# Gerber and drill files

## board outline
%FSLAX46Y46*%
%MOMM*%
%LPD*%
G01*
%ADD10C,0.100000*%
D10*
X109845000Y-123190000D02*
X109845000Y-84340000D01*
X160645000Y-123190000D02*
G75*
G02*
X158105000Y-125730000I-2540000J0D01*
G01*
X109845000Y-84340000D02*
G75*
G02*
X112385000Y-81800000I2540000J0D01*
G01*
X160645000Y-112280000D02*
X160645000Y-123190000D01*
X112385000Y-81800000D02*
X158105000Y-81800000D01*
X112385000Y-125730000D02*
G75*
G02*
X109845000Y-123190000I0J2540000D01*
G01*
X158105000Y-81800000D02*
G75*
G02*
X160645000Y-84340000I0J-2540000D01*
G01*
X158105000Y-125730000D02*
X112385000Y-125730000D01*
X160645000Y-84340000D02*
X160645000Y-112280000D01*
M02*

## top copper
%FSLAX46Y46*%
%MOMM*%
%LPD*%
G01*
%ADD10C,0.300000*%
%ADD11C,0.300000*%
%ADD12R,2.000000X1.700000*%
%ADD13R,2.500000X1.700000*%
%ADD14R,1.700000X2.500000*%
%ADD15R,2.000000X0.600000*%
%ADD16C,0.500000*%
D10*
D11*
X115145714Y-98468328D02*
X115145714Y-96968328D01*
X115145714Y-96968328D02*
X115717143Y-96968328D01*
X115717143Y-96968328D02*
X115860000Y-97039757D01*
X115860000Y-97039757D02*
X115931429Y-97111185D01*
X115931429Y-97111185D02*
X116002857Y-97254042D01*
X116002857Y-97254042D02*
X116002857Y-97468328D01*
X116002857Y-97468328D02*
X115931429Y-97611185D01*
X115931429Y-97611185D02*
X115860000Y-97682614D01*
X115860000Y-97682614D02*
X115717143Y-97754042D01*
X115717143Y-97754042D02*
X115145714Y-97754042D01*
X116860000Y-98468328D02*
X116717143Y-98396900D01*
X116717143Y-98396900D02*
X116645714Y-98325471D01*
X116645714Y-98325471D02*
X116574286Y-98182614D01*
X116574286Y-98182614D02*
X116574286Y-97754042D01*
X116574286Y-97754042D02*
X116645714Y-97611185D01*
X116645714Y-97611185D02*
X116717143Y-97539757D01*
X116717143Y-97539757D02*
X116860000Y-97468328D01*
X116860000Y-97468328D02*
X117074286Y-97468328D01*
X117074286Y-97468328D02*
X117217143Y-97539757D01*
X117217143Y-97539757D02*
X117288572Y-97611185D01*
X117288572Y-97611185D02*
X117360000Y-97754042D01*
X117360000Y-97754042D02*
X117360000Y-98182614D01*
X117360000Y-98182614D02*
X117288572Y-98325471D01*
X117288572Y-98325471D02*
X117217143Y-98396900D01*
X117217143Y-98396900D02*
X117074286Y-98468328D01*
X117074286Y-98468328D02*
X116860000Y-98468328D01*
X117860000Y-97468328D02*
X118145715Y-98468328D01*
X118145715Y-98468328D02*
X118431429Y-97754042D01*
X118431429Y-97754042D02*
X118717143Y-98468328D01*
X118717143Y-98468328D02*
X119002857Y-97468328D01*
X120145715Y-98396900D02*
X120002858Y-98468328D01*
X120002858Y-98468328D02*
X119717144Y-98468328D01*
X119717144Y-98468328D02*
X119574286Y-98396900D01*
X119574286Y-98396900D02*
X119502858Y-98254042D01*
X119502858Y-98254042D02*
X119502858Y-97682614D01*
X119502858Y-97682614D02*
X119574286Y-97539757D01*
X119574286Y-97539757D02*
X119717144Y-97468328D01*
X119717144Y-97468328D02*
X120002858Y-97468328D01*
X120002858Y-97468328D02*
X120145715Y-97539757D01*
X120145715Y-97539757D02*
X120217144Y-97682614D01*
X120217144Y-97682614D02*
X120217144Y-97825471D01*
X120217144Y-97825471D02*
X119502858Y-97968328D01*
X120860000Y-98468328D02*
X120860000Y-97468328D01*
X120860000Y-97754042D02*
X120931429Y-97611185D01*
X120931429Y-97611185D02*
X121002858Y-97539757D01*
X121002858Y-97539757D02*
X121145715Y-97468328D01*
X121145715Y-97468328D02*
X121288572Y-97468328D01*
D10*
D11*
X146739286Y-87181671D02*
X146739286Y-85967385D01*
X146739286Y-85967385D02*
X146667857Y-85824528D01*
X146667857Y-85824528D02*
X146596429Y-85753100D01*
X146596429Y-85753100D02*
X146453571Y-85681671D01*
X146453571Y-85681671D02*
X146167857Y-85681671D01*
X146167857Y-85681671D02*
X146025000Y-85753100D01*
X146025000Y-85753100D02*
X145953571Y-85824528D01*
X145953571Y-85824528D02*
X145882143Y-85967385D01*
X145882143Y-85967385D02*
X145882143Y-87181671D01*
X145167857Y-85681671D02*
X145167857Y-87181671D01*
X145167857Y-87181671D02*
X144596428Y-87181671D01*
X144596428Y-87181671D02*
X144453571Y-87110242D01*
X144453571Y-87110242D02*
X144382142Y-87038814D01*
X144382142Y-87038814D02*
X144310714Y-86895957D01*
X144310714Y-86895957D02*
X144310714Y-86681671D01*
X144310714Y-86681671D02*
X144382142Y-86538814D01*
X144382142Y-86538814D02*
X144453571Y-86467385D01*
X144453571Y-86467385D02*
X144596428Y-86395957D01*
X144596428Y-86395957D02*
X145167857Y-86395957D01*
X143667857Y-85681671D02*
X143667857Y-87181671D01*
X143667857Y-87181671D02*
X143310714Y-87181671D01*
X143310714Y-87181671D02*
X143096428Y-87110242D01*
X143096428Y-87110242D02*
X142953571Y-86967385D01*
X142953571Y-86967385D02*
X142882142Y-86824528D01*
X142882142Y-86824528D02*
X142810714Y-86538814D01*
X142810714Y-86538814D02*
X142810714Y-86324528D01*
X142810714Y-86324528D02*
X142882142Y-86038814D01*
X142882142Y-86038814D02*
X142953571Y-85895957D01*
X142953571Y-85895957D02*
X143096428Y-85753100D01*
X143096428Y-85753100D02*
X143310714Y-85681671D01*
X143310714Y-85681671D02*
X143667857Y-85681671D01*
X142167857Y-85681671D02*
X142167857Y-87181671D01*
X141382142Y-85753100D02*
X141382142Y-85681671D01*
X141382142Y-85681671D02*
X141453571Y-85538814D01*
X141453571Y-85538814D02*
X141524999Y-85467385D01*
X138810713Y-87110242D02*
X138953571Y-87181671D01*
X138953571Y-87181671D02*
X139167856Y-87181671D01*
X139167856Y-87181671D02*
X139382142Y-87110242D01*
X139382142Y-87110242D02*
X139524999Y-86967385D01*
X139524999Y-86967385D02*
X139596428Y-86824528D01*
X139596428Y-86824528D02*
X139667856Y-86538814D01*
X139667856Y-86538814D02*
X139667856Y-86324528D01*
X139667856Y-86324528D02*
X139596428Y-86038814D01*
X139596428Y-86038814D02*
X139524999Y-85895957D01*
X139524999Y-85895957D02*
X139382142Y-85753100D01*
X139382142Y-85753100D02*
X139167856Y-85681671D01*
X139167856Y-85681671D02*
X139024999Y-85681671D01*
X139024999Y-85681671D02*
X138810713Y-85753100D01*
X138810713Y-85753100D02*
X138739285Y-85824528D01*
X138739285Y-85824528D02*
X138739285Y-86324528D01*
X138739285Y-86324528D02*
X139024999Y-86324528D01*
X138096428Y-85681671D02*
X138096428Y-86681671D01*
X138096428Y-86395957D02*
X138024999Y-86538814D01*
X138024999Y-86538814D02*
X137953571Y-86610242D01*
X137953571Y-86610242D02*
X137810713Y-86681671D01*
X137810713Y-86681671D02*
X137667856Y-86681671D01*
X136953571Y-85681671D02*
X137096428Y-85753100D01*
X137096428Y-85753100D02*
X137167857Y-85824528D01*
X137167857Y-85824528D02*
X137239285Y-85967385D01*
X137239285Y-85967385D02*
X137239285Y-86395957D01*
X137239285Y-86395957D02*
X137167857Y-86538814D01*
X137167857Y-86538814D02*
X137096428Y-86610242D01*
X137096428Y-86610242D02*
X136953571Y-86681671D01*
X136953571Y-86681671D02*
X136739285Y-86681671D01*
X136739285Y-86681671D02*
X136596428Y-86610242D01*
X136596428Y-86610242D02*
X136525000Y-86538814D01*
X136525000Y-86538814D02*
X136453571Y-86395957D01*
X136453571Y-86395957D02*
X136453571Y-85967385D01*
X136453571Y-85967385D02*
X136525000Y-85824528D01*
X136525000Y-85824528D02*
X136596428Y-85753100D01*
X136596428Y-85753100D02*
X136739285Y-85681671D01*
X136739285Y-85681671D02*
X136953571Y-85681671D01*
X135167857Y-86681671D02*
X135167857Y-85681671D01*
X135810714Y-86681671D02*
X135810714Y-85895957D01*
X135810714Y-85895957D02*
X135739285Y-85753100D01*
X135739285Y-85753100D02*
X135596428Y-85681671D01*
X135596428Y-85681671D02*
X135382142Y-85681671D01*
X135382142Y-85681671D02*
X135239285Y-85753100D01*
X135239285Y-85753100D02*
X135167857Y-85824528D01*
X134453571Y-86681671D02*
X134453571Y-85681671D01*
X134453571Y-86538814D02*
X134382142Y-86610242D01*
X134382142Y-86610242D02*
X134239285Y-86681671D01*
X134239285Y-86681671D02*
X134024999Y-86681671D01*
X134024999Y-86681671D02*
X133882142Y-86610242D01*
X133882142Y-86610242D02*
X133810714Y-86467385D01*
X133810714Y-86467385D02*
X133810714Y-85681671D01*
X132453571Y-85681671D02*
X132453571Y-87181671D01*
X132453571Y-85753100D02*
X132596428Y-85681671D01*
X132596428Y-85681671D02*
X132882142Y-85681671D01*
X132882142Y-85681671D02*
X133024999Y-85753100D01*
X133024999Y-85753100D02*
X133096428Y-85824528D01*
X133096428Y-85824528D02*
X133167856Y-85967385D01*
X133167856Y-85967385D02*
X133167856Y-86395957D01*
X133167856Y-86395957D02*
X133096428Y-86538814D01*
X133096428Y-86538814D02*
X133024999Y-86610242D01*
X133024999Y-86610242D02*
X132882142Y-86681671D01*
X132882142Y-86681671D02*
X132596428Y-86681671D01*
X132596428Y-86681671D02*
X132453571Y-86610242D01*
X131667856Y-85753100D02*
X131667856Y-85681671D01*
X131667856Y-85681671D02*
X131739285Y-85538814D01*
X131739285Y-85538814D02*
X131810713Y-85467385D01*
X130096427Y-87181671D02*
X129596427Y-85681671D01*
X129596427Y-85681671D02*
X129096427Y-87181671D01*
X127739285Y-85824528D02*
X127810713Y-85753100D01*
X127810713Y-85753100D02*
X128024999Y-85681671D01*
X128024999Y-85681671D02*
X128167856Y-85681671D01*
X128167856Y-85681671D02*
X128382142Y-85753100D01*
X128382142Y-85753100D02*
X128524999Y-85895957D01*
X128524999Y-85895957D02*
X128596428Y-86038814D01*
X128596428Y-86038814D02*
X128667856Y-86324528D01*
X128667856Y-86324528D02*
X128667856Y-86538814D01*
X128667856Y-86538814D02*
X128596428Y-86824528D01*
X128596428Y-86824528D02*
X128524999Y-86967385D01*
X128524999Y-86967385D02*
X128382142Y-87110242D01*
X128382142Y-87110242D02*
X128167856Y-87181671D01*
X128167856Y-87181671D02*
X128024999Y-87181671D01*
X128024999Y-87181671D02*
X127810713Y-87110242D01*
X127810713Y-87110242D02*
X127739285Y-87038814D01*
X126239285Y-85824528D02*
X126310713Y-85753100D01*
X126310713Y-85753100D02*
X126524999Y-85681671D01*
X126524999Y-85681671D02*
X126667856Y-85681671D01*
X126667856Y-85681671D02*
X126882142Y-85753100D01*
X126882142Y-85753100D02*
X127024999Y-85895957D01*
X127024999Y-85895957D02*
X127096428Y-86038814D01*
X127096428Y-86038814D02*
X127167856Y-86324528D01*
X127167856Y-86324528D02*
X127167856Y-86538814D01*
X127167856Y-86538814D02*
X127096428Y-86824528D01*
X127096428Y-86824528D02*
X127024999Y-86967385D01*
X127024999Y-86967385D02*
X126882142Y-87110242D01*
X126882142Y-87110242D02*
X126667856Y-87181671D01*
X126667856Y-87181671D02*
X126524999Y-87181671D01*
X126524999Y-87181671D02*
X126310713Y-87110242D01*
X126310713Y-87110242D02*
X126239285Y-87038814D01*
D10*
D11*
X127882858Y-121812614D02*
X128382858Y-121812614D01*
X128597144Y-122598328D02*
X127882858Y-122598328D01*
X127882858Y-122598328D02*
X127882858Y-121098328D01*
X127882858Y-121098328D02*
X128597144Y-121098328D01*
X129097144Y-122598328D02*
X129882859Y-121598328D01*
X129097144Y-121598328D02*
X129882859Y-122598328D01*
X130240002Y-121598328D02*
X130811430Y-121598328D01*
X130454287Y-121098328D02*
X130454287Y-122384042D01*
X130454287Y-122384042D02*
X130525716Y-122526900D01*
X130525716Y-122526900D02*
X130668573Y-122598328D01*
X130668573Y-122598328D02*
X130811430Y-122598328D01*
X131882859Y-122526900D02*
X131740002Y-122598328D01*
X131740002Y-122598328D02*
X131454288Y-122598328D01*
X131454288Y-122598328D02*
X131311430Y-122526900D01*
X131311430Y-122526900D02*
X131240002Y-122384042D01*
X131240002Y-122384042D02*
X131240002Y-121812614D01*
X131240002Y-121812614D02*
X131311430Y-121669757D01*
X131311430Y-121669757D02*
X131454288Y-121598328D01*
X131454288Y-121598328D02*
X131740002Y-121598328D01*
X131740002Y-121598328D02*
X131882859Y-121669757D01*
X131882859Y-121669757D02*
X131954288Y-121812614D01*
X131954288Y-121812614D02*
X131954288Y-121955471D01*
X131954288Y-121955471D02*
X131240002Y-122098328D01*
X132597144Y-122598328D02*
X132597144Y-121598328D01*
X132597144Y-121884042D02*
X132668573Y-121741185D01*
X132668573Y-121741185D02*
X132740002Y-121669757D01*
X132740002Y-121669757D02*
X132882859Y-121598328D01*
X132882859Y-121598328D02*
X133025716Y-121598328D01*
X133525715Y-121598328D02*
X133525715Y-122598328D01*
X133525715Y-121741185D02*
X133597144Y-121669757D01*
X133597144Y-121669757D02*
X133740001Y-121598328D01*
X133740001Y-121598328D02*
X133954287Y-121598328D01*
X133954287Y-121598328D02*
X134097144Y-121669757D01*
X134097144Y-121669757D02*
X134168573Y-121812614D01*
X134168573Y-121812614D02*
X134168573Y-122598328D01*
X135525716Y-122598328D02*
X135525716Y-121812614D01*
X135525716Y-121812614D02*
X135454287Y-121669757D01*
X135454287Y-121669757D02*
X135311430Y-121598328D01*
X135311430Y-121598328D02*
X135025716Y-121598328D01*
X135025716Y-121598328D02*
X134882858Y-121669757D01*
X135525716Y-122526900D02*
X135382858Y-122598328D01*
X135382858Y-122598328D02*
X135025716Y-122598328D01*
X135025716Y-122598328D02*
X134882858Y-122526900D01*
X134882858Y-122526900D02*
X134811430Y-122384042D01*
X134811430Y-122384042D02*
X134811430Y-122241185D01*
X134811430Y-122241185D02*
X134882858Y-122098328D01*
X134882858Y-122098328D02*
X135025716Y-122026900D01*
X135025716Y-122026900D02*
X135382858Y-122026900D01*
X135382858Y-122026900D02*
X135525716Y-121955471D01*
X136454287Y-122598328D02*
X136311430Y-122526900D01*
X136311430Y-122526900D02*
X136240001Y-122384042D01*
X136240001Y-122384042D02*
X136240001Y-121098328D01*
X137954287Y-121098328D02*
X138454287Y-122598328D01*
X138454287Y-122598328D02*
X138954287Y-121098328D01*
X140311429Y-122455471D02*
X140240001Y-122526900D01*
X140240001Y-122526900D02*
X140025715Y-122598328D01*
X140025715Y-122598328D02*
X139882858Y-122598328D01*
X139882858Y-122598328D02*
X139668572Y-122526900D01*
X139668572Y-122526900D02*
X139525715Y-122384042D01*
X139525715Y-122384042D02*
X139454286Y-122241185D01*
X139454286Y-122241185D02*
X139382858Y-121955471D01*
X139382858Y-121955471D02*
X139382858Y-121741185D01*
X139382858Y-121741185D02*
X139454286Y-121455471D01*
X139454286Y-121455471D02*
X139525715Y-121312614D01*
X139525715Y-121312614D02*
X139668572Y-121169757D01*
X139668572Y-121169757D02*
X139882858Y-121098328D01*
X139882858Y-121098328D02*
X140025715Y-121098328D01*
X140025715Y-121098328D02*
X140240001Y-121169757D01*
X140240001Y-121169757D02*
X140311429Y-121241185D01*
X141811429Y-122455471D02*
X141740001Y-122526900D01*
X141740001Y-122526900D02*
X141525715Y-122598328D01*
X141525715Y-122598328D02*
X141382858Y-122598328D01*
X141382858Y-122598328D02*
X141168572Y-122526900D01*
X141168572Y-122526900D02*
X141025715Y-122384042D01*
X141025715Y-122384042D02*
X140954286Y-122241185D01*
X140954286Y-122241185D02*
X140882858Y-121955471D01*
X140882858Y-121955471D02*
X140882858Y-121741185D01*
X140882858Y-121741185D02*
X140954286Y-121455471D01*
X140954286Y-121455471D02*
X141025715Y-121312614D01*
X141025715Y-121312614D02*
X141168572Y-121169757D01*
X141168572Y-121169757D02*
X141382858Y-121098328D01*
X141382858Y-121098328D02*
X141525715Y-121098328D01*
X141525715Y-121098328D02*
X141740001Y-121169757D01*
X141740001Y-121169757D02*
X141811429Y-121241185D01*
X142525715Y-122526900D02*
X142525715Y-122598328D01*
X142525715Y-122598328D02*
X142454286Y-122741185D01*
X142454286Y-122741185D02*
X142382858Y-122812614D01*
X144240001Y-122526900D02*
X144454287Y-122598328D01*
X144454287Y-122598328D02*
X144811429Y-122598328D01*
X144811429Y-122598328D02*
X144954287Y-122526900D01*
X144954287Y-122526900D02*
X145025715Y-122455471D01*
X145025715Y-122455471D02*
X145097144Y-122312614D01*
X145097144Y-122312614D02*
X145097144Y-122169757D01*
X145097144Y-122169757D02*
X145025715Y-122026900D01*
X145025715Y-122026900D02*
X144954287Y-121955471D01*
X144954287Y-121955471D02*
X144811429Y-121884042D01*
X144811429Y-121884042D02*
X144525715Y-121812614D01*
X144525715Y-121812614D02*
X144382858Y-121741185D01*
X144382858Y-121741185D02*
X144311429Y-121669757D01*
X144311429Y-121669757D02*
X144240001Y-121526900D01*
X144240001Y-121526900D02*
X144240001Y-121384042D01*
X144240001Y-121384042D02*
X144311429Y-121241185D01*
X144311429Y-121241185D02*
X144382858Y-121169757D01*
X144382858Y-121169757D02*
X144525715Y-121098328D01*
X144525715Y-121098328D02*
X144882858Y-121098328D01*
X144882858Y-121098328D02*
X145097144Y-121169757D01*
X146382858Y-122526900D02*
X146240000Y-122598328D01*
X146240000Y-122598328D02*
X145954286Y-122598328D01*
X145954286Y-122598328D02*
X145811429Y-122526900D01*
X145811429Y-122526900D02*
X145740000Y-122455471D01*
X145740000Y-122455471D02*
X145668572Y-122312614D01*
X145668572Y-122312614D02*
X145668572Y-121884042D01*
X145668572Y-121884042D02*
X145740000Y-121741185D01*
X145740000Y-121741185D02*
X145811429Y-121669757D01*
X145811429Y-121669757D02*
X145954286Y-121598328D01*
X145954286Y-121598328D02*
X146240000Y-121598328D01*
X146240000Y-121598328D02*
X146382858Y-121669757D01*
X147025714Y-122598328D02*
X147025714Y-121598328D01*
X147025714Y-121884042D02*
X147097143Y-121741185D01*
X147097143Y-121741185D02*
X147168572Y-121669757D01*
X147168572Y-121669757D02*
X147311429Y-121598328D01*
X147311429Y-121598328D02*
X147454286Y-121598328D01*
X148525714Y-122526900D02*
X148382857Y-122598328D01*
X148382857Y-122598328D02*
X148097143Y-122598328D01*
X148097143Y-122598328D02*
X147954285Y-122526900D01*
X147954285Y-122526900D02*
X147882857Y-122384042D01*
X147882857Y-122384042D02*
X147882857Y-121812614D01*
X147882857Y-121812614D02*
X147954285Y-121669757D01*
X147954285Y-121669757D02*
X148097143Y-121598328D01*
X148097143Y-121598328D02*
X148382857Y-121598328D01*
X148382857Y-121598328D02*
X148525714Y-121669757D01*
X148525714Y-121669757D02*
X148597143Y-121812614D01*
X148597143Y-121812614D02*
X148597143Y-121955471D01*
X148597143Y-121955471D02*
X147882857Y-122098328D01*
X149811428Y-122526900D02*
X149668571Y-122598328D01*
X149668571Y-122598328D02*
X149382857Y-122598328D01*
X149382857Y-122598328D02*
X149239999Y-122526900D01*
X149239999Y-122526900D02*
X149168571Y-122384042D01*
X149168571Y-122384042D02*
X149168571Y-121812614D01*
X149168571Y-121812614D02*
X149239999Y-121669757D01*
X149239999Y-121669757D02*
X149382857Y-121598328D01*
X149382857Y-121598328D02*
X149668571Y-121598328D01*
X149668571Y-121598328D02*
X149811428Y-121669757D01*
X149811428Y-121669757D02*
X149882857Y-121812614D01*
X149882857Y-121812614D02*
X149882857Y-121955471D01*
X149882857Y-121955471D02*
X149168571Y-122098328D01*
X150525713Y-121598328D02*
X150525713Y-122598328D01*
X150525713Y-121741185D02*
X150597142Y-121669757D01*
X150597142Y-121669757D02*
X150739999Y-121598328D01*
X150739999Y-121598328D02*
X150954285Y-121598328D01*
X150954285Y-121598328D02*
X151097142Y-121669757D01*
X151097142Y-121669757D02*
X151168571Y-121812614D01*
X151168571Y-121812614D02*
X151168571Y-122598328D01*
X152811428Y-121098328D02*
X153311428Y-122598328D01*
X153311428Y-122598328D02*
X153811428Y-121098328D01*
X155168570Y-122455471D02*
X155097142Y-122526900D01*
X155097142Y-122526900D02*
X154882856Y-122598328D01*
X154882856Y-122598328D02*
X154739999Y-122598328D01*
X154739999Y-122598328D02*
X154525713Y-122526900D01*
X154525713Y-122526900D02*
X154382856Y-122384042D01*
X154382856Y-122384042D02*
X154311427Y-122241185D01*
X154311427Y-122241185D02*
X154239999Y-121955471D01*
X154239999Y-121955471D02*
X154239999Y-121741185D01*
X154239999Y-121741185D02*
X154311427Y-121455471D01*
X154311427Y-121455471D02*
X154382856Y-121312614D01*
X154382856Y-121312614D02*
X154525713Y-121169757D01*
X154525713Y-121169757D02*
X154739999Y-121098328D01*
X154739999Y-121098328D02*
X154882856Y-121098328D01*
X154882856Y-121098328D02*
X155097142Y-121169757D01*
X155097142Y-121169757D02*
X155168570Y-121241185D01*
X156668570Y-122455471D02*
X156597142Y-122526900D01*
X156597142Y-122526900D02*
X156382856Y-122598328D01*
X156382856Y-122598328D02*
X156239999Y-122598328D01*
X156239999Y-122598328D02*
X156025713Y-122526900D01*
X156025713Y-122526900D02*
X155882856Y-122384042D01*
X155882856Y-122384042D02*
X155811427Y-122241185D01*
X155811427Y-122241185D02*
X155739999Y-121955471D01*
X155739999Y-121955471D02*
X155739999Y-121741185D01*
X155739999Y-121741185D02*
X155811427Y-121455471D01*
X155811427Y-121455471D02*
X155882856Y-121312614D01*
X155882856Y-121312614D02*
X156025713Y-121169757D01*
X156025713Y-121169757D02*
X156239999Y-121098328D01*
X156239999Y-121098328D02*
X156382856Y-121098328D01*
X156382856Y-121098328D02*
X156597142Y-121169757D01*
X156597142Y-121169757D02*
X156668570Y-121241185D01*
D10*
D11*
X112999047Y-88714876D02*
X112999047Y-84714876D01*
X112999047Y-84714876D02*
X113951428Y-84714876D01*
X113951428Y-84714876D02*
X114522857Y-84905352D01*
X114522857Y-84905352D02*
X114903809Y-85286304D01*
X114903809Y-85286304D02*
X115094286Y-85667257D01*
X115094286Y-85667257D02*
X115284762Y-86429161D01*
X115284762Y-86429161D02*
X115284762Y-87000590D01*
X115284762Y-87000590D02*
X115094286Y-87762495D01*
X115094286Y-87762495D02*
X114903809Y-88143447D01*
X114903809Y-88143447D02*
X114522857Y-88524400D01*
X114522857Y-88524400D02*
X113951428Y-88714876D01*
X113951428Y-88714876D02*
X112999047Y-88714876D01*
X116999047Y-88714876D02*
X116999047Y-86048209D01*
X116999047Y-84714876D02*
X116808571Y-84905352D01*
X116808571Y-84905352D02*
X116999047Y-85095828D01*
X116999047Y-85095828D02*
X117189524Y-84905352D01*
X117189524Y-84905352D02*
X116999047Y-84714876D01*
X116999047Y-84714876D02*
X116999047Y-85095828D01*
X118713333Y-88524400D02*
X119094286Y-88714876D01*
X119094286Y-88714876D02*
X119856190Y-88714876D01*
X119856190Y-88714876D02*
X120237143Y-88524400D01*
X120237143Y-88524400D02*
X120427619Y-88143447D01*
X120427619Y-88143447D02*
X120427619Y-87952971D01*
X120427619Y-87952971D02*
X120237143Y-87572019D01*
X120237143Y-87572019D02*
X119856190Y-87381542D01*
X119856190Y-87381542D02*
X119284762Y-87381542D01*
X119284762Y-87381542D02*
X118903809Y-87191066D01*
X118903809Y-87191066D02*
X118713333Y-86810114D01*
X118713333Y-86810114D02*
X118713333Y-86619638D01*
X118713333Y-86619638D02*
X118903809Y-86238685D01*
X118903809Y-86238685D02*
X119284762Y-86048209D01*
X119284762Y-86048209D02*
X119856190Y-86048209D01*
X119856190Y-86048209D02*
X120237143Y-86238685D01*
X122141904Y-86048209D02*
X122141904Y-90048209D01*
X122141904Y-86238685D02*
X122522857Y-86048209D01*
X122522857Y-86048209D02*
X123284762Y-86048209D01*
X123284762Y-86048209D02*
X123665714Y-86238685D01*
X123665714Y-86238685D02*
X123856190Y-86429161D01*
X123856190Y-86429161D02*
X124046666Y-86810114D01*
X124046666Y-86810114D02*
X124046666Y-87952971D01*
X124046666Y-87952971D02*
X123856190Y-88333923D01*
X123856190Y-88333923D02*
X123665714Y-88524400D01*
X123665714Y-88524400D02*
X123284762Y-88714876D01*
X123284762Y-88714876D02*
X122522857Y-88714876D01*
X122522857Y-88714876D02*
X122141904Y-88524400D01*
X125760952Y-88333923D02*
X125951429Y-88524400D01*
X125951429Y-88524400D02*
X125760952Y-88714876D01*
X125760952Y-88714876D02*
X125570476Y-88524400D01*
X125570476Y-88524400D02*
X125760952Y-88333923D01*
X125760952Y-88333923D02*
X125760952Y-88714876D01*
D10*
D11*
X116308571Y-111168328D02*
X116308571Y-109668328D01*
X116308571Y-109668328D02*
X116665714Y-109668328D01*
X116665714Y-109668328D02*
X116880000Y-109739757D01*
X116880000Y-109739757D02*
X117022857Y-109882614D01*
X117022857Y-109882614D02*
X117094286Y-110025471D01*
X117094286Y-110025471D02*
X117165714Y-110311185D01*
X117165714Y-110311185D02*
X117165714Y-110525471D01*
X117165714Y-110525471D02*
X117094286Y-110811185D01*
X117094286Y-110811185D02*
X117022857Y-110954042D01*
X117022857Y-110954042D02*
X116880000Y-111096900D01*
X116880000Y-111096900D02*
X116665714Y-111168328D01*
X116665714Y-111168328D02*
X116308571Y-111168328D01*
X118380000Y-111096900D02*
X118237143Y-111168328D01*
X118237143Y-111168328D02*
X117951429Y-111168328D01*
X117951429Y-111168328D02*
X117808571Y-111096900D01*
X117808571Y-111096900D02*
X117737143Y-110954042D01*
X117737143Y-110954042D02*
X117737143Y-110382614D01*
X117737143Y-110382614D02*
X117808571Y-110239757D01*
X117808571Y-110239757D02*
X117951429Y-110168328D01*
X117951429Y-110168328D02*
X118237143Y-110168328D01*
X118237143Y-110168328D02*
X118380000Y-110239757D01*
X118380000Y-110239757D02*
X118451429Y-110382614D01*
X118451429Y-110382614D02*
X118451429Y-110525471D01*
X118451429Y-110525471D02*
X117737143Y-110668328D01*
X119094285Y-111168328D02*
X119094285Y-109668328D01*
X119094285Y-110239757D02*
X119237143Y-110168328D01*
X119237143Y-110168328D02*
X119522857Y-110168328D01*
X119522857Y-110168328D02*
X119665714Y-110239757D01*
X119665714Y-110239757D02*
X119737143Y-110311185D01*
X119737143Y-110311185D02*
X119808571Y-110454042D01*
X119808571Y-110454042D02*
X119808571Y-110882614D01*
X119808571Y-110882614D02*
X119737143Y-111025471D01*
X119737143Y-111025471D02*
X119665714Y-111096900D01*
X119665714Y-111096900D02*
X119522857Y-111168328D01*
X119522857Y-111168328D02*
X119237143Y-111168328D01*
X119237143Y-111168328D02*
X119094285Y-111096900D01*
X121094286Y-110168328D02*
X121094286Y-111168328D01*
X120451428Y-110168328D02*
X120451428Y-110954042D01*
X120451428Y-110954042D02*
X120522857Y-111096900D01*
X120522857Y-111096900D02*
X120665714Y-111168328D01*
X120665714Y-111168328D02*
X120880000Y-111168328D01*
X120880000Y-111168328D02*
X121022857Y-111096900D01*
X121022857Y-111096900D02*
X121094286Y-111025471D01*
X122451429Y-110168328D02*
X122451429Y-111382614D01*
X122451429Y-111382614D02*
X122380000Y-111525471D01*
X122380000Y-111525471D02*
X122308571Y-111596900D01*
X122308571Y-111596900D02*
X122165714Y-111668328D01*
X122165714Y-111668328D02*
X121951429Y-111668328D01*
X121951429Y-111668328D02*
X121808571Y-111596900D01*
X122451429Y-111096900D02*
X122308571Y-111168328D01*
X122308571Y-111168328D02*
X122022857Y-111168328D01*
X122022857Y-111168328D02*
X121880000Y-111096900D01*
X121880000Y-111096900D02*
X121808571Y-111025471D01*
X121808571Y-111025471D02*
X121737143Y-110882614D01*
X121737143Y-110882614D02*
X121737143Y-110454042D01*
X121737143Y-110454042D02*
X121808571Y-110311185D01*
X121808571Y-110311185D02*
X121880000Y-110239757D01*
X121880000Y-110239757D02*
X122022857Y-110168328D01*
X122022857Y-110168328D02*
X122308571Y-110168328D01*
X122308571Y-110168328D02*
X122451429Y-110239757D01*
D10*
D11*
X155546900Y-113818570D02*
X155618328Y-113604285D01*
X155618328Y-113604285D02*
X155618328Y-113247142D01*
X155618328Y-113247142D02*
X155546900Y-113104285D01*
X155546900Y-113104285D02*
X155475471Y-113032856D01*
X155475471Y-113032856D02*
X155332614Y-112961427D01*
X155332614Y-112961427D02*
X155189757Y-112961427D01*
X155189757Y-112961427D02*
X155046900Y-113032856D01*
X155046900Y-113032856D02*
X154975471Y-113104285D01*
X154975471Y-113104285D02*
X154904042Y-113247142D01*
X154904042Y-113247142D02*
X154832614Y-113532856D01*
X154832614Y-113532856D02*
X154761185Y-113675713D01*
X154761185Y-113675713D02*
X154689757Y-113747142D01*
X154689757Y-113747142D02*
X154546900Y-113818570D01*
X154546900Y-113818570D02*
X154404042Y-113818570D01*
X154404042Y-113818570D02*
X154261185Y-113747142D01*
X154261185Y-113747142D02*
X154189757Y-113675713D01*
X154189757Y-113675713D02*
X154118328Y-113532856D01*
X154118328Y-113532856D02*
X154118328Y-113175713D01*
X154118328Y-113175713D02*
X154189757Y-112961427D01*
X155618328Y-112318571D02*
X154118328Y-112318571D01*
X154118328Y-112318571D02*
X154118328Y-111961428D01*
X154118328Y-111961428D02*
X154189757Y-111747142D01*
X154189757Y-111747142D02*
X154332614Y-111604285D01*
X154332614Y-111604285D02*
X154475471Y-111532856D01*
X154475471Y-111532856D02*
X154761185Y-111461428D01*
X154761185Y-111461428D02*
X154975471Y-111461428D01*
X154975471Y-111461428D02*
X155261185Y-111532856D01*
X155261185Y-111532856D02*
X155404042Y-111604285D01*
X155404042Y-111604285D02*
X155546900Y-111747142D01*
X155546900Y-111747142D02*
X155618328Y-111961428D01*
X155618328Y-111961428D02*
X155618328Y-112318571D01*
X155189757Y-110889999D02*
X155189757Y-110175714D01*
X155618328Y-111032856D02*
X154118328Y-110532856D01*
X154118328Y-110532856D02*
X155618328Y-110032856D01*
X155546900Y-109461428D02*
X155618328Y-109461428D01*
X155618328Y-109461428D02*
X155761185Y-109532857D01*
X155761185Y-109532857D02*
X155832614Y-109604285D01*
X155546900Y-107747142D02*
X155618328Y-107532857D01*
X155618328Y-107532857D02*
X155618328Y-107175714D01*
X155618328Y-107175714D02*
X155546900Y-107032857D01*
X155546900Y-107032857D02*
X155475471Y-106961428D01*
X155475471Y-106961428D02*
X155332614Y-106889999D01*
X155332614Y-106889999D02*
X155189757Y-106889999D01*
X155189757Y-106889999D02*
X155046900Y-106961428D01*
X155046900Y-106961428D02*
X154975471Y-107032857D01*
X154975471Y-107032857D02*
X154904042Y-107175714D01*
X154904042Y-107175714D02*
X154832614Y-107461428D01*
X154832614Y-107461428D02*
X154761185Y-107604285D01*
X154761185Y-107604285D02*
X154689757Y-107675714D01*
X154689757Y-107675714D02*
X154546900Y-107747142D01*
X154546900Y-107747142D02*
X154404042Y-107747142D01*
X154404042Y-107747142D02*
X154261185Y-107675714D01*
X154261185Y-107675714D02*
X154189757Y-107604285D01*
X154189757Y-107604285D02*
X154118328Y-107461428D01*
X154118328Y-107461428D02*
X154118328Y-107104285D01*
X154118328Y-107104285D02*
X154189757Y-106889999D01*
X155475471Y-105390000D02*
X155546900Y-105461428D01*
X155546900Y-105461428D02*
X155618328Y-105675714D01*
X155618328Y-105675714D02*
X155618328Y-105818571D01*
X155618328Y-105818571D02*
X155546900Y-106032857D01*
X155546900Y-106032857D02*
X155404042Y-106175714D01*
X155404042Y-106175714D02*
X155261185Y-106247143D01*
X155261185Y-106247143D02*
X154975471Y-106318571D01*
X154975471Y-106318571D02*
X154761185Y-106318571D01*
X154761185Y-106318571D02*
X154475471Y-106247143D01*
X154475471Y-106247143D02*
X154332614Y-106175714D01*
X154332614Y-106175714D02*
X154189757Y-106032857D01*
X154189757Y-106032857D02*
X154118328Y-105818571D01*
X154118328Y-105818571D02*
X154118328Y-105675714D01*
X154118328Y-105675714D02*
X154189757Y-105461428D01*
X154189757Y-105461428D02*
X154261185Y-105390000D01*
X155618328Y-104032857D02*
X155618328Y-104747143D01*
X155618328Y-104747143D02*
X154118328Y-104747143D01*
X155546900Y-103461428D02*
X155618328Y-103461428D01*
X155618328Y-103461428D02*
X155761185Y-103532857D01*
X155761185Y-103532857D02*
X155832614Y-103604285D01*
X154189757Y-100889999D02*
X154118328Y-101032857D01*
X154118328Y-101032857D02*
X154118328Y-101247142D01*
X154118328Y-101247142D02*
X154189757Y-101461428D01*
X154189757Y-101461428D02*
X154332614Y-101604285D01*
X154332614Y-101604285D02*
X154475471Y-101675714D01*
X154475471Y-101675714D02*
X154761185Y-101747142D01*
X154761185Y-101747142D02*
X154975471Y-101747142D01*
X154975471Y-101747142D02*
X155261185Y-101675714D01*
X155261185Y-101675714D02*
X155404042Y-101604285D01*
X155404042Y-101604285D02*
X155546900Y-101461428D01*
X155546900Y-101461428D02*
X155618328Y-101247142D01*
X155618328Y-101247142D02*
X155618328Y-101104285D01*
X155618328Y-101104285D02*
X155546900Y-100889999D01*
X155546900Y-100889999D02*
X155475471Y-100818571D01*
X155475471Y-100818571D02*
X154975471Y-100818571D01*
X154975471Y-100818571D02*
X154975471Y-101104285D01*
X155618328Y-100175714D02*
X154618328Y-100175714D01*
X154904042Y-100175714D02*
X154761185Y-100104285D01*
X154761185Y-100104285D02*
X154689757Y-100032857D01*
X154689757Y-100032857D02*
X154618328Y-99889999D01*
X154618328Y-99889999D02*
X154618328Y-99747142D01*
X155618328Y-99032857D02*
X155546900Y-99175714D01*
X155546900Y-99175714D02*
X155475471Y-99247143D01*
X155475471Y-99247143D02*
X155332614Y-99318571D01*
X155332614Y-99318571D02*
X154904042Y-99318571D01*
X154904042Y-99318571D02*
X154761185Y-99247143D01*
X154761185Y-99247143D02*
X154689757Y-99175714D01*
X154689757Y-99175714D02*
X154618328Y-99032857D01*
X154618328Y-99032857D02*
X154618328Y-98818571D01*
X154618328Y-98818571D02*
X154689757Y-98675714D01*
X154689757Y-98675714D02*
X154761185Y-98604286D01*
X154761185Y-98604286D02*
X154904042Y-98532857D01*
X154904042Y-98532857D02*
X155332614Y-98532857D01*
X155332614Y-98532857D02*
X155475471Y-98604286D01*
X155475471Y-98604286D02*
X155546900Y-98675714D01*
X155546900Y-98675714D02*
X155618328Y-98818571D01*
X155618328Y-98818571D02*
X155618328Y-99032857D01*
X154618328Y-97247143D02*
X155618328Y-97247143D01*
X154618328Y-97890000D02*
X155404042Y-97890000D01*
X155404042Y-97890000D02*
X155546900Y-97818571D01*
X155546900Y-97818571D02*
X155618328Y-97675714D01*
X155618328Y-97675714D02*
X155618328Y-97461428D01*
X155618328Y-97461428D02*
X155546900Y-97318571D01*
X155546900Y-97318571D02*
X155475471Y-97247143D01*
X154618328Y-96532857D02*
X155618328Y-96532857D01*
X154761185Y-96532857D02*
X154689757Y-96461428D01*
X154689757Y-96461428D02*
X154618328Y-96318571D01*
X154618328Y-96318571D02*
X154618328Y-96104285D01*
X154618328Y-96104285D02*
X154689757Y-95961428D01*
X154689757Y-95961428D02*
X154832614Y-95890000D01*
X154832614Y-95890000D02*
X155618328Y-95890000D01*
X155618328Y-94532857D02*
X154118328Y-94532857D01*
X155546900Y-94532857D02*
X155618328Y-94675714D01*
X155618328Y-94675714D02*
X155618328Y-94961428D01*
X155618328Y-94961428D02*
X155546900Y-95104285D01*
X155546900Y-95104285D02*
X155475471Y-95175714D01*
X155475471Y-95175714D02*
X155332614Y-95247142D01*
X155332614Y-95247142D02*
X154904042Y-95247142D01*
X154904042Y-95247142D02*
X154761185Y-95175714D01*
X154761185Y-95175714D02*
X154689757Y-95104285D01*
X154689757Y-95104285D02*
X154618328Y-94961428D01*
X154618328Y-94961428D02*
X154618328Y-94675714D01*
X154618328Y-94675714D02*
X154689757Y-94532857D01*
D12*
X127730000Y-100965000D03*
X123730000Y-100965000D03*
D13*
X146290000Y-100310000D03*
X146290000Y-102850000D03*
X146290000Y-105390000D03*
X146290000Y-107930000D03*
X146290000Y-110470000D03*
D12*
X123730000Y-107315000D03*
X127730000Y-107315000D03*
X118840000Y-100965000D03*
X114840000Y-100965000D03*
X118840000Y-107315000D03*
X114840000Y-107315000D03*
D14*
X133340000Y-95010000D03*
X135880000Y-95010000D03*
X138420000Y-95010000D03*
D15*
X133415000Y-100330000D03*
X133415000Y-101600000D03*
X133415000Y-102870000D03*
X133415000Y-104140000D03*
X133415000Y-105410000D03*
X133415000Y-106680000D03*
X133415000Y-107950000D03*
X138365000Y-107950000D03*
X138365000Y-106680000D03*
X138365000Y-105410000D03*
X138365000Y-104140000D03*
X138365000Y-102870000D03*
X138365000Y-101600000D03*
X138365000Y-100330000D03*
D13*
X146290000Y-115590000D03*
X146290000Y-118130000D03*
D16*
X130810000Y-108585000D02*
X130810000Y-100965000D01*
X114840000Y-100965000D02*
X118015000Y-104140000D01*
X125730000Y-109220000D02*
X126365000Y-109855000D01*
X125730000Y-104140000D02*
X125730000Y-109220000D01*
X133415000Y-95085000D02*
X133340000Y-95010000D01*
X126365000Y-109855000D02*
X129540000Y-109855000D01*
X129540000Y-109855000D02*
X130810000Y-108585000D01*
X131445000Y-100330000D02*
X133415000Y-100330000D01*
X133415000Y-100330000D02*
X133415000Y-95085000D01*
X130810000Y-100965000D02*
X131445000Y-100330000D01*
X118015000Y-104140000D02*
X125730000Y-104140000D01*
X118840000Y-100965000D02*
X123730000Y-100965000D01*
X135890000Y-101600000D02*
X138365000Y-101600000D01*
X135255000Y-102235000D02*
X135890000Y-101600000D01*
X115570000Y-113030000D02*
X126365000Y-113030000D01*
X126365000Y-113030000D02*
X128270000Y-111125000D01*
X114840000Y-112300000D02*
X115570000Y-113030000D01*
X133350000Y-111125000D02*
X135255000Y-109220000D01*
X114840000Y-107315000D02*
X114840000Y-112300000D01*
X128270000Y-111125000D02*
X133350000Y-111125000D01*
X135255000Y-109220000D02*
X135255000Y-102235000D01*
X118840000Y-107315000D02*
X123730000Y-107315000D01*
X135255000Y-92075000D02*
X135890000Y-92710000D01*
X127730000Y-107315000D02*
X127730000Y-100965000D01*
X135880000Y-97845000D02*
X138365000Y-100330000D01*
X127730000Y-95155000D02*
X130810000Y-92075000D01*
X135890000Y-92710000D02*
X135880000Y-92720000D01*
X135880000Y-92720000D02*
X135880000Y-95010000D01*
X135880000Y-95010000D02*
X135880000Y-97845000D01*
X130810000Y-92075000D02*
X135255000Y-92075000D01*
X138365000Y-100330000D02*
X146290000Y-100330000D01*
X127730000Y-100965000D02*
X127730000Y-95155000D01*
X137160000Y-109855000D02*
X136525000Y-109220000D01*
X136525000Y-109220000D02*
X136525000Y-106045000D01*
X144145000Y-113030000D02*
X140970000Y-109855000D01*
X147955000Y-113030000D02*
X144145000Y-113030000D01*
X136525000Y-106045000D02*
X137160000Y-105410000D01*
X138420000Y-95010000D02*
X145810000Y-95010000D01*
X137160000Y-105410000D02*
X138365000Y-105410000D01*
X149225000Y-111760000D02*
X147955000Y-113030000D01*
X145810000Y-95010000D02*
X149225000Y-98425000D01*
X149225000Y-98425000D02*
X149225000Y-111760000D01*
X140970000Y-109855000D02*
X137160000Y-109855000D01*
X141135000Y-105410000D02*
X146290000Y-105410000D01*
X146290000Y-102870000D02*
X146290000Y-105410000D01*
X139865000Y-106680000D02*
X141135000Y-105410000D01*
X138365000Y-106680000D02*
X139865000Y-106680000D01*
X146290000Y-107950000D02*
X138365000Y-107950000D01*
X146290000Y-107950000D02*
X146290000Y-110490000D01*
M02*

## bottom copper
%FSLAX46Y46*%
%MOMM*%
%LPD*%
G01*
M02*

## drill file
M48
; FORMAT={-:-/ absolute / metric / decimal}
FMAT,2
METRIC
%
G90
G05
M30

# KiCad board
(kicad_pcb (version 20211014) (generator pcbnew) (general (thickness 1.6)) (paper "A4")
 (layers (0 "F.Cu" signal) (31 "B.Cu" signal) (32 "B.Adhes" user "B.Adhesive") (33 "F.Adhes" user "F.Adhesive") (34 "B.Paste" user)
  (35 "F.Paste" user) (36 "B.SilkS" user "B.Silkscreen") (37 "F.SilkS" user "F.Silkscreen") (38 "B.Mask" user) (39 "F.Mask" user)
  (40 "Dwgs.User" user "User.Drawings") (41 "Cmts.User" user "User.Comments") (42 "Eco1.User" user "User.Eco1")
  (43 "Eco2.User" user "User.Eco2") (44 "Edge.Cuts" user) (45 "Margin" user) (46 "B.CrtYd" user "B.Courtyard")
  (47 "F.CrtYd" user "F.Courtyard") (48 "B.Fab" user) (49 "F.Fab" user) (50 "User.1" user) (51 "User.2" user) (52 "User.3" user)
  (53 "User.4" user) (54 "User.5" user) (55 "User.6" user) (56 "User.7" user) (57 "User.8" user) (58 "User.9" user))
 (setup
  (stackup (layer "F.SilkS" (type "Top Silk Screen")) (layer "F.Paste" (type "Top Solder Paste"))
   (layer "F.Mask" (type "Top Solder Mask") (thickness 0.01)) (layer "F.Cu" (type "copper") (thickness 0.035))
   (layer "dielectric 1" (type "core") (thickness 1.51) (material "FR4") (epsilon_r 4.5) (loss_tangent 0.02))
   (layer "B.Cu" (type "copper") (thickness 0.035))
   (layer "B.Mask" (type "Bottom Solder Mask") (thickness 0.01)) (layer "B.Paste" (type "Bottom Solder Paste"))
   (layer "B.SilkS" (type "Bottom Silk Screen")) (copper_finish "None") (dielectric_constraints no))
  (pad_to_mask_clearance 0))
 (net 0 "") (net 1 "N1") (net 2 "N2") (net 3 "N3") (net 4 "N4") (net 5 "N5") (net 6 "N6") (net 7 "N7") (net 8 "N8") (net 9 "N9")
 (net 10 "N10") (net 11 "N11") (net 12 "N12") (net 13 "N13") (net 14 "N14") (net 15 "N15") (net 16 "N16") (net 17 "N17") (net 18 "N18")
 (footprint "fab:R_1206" (layer "F.Cu") (at 125.73 100.965 180)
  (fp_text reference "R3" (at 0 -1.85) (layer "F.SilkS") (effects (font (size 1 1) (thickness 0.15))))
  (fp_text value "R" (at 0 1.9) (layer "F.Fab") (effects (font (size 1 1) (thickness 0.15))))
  (pad "1" smd rect locked (at -2 0 180) (size 2 1.7) (layers "F.Cu" "F.Paste" "F.Mask") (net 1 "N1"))
  (pad "2" smd rect locked (at 2 0 180) (size 2 1.7) (layers "F.Cu" "F.Paste" "F.Mask") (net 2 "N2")))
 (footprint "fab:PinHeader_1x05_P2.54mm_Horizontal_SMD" (layer "F.Cu") (at 146.29 100.31)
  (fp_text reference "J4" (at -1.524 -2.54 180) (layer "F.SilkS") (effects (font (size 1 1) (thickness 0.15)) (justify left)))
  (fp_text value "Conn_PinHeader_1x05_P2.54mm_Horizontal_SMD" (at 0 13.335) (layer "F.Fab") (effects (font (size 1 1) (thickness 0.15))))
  (pad "1" smd rect locked (at 0 0) (size 2.5 1.7) (layers "F.Cu" "F.Paste" "F.Mask") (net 1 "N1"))
  (pad "2" smd rect locked (at 0 2.54) (size 2.5 1.7) (layers "F.Cu" "F.Paste" "F.Mask") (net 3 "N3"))
  (pad "3" smd rect locked (at 0 5.08) (size 2.5 1.7) (layers "F.Cu" "F.Paste" "F.Mask") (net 3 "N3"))
  (pad "4" smd rect locked (at 0 7.62) (size 2.5 1.7) (layers "F.Cu" "F.Paste" "F.Mask") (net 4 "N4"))
  (pad "5" smd rect locked (at 0 10.16) (size 2.5 1.7) (layers "F.Cu" "F.Paste" "F.Mask") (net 4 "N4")))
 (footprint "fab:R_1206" (layer "F.Cu") (at 125.73 107.315)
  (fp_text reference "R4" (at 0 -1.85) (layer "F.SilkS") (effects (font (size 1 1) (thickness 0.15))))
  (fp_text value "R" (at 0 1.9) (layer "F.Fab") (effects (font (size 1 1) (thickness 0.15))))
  (pad "1" smd rect locked (at -2 0) (size 2 1.7) (layers "F.Cu" "F.Paste" "F.Mask") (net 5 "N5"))
  (pad "2" smd rect locked (at 2 0) (size 2 1.7) (layers "F.Cu" "F.Paste" "F.Mask") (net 1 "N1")))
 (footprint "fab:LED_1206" (layer "F.Cu") (at 116.84 100.965 180)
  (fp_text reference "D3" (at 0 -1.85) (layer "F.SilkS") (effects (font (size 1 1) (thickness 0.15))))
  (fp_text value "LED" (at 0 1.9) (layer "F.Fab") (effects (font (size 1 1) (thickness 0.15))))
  (pad "1" smd rect locked (at -2 0 180) (size 2 1.7) (layers "F.Cu" "F.Paste" "F.Mask") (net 2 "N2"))
  (pad "2" smd rect locked (at 2 0 180) (size 2 1.7) (layers "F.Cu" "F.Paste" "F.Mask") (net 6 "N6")))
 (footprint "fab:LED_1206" (layer "F.Cu") (at 116.84 107.315 180)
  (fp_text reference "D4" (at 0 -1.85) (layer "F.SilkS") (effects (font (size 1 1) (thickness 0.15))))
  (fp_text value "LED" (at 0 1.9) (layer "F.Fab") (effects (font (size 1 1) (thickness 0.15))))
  (pad "1" smd rect locked (at -2 0 180) (size 2 1.7) (layers "F.Cu" "F.Paste" "F.Mask") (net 5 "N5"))
  (pad "2" smd rect locked (at 2 0 180) (size 2 1.7) (layers "F.Cu" "F.Paste" "F.Mask") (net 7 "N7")))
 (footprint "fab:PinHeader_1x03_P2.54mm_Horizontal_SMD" (layer "F.Cu") (at 133.34 95.01 90)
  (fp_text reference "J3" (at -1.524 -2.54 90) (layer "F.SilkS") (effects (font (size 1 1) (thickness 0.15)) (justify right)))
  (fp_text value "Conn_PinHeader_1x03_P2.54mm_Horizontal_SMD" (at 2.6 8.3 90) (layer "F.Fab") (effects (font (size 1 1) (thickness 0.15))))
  (pad "1" smd rect locked (at 0 0 90) (size 2.5 1.7) (layers "F.Cu" "F.Paste" "F.Mask") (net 6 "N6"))
  (pad "2" smd rect locked (at 0 2.54 90) (size 2.5 1.7) (layers "F.Cu" "F.Paste" "F.Mask") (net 1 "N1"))
  (pad "3" smd rect locked (at 0 5.08 90) (size 2.5 1.7) (layers "F.Cu" "F.Paste" "F.Mask") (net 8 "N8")))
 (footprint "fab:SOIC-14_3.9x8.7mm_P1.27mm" (layer "F.Cu") (at 135.89 104.14)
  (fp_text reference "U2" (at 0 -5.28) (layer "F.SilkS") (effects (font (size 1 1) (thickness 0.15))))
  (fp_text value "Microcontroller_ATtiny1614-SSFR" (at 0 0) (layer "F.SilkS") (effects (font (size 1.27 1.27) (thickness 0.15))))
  (pad "1" smd rect (at -2.475 -3.81) (size 2 0.6) (layers "F.Cu" "F.Paste" "F.Mask") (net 6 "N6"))
  (pad "2" smd rect (at -2.475 -2.54) (size 2 0.6) (layers "F.Cu" "F.Paste" "F.Mask") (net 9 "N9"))
  (pad "3" smd rect (at -2.475 -1.27) (size 2 0.6) (layers "F.Cu" "F.Paste" "F.Mask") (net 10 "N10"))
  (pad "4" smd rect (at -2.475 0) (size 2 0.6) (layers "F.Cu" "F.Paste" "F.Mask") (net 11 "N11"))
  (pad "5" smd rect (at -2.475 1.27) (size 2 0.6) (layers "F.Cu" "F.Paste" "F.Mask") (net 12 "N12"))
  (pad "6" smd rect (at -2.475 2.54) (size 2 0.6) (layers "F.Cu" "F.Paste" "F.Mask") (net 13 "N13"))
  (pad "7" smd rect (at -2.475 3.81) (size 2 0.6) (layers "F.Cu" "F.Paste" "F.Mask") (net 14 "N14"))
  (pad "8" smd rect (at 2.475 3.81) (size 2 0.6) (layers "F.Cu" "F.Paste" "F.Mask") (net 4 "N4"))
  (pad "9" smd rect (at 2.475 2.54) (size 2 0.6) (layers "F.Cu" "F.Paste" "F.Mask") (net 3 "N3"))
  (pad "10" smd rect (at 2.475 1.27) (size 2 0.6) (layers "F.Cu" "F.Paste" "F.Mask") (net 8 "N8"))
  (pad "11" smd rect (at 2.475 0) (size 2 0.6) (layers "F.Cu" "F.Paste" "F.Mask") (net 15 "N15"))
  (pad "12" smd rect (at 2.475 -1.27) (size 2 0.6) (layers "F.Cu" "F.Paste" "F.Mask") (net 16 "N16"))
  (pad "13" smd rect (at 2.475 -2.54) (size 2 0.6) (layers "F.Cu" "F.Paste" "F.Mask") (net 7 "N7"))
  (pad "14" smd rect (at 2.475 -3.81) (size 2 0.6) (layers "F.Cu" "F.Paste" "F.Mask") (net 1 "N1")))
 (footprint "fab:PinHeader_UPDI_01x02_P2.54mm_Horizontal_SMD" (layer "F.Cu") (at 146.29 115.59)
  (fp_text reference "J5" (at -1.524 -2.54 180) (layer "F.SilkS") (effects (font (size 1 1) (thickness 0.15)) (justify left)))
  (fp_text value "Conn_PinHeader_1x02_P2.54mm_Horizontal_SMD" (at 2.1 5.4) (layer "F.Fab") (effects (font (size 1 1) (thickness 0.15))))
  (pad "1" smd rect locked (at 0 0) (size 2.5 1.7) (layers "F.Cu" "F.Paste" "F.Mask") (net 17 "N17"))
  (pad "2" smd rect locked (at 0 2.54) (size 2.5 1.7) (layers "F.Cu" "F.Paste" "F.Mask") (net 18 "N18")))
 (gr_line (start 109.845 123.19) (end 109.845 84.34) (layer "Edge.Cuts") (width 0.1))
 (gr_arc (start 160.645 123.19) (mid 159.901051 124.986051) (end 158.105 125.73) (layer "Edge.Cuts") (width 0.1))
 (gr_arc (start 109.845 84.34) (mid 110.588949 82.543949) (end 112.385 81.8) (layer "Edge.Cuts") (width 0.1))
 (gr_line (start 160.645 112.28) (end 160.645 123.19) (layer "Edge.Cuts") (width 0.1))
 (gr_line (start 112.385 81.8) (end 158.105 81.8) (layer "Edge.Cuts") (width 0.1))
 (gr_arc (start 112.385 125.73) (mid 110.588949 124.986051) (end 109.845 123.19) (layer "Edge.Cuts") (width 0.1))
 (gr_arc (start 158.105 81.8) (mid 159.901051 82.543949) (end 160.645 84.34) (layer "Edge.Cuts") (width 0.1))
 (gr_line (start 158.105 125.73) (end 112.385 125.73) (layer "Edge.Cuts") (width 0.1))
 (gr_line (start 160.645 84.34) (end 160.645 112.28) (layer "Edge.Cuts") (width 0.1))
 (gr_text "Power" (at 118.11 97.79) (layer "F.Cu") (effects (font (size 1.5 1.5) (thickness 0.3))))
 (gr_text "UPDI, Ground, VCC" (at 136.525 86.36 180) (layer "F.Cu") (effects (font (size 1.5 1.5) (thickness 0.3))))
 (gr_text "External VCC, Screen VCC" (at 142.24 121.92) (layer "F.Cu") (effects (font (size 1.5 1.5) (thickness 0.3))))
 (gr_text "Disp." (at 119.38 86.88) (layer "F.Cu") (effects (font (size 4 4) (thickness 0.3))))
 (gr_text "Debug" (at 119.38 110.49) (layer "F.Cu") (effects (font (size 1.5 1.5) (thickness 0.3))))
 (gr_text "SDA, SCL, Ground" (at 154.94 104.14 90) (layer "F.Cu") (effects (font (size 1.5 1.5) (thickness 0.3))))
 (segment (start 130.81 108.585) (end 130.81 100.965) (width 0.5) (layer "F.Cu") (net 6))
 (segment (start 114.84 100.965) (end 118.015 104.14) (width 0.5) (layer "F.Cu") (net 6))
 (segment (start 125.73 109.22) (end 126.365 109.855) (width 0.5) (layer "F.Cu") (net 6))
 (segment (start 125.73 104.14) (end 125.73 109.22) (width 0.5) (layer "F.Cu") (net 6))
 (segment (start 133.415 95.085) (end 133.34 95.01) (width 0.5) (layer "F.Cu") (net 6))
 (segment (start 126.365 109.855) (end 129.54 109.855) (width 0.5) (layer "F.Cu") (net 6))
 (segment (start 129.54 109.855) (end 130.81 108.585) (width 0.5) (layer "F.Cu") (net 6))
 (segment (start 131.445 100.33) (end 133.415 100.33) (width 0.5) (layer "F.Cu") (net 6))
 (segment (start 133.415 100.33) (end 133.415 95.085) (width 0.5) (layer "F.Cu") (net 6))
 (segment (start 130.81 100.965) (end 131.445 100.33) (width 0.5) (layer "F.Cu") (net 6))
 (segment (start 118.015 104.14) (end 125.73 104.14) (width 0.5) (layer "F.Cu") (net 6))
 (segment (start 118.84 100.965) (end 123.73 100.965) (width 0.5) (layer "F.Cu") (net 2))
 (segment (start 135.89 101.6) (end 138.365 101.6) (width 0.5) (layer "F.Cu") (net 7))
 (segment (start 135.255 102.235) (end 135.89 101.6) (width 0.5) (layer "F.Cu") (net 7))
 (segment (start 115.57 113.03) (end 126.365 113.03) (width 0.5) (layer "F.Cu") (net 7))
 (segment (start 126.365 113.03) (end 128.27 111.125) (width 0.5) (layer "F.Cu") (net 7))
 (segment (start 114.84 112.3) (end 115.57 113.03) (width 0.5) (layer "F.Cu") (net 7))
 (segment (start 133.35 111.125) (end 135.255 109.22) (width 0.5) (layer "F.Cu") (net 7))
 (segment (start 114.84 107.315) (end 114.84 112.3) (width 0.5) (layer "F.Cu") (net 7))
 (segment (start 128.27 111.125) (end 133.35 111.125) (width 0.5) (layer "F.Cu") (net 7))
 (segment (start 135.255 109.22) (end 135.255 102.235) (width 0.5) (layer "F.Cu") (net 7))
 (segment (start 118.84 107.315) (end 123.73 107.315) (width 0.5) (layer "F.Cu") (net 5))
 (segment (start 135.255 92.075) (end 135.89 92.71) (width 0.5) (layer "F.Cu") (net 1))
 (segment (start 127.73 107.315) (end 127.73 100.965) (width 0.5) (layer "F.Cu") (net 1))
 (segment (start 135.88 97.845) (end 138.365 100.33) (width 0.5) (layer "F.Cu") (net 1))
 (segment (start 127.73 95.155) (end 130.81 92.075) (width 0.5) (layer "F.Cu") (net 1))
 (segment (start 135.89 92.71) (end 135.88 92.72) (width 0.5) (layer "F.Cu") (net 1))
 (segment (start 135.88 92.72) (end 135.88 95.01) (width 0.5) (layer "F.Cu") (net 1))
 (segment (start 135.88 95.01) (end 135.88 97.845) (width 0.5) (layer "F.Cu") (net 1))
 (segment (start 130.81 92.075) (end 135.255 92.075) (width 0.5) (layer "F.Cu") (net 1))
 (segment (start 138.365 100.33) (end 146.29 100.33) (width 0.5) (layer "F.Cu") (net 1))
 (segment (start 127.73 100.965) (end 127.73 95.155) (width 0.5) (layer "F.Cu") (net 1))
 (segment (start 137.16 109.855) (end 136.525 109.22) (width 0.5) (layer "F.Cu") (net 8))
 (segment (start 136.525 109.22) (end 136.525 106.045) (width 0.5) (layer "F.Cu") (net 8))
 (segment (start 144.145 113.03) (end 140.97 109.855) (width 0.5) (layer "F.Cu") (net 8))
 (segment (start 147.955 113.03) (end 144.145 113.03) (width 0.5) (layer "F.Cu") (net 8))
 (segment (start 136.525 106.045) (end 137.16 105.41) (width 0.5) (layer "F.Cu") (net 8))
 (segment (start 138.42 95.01) (end 145.81 95.01) (width 0.5) (layer "F.Cu") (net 8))
 (segment (start 137.16 105.41) (end 138.365 105.41) (width 0.5) (layer "F.Cu") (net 8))
 (segment (start 149.225 111.76) (end 147.955 113.03) (width 0.5) (layer "F.Cu") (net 8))
 (segment (start 145.81 95.01) (end 149.225 98.425) (width 0.5) (layer "F.Cu") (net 8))
 (segment (start 149.225 98.425) (end 149.225 111.76) (width 0.5) (layer "F.Cu") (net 8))
 (segment (start 140.97 109.855) (end 137.16 109.855) (width 0.5) (layer "F.Cu") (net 8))
 (segment (start 141.135 105.41) (end 146.29 105.41) (width 0.5) (layer "F.Cu") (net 3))
 (segment (start 146.29 102.87) (end 146.29 105.41) (width 0.5) (layer "F.Cu") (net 3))
 (segment (start 139.865 106.68) (end 141.135 105.41) (width 0.5) (layer "F.Cu") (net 3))
 (segment (start 138.365 106.68) (end 139.865 106.68) (width 0.5) (layer "F.Cu") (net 3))
 (segment (start 146.29 107.95) (end 138.365 107.95) (width 0.5) (layer "F.Cu") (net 4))
 (segment (start 146.29 107.95) (end 146.29 110.49) (width 0.5) (layer "F.Cu") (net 4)))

